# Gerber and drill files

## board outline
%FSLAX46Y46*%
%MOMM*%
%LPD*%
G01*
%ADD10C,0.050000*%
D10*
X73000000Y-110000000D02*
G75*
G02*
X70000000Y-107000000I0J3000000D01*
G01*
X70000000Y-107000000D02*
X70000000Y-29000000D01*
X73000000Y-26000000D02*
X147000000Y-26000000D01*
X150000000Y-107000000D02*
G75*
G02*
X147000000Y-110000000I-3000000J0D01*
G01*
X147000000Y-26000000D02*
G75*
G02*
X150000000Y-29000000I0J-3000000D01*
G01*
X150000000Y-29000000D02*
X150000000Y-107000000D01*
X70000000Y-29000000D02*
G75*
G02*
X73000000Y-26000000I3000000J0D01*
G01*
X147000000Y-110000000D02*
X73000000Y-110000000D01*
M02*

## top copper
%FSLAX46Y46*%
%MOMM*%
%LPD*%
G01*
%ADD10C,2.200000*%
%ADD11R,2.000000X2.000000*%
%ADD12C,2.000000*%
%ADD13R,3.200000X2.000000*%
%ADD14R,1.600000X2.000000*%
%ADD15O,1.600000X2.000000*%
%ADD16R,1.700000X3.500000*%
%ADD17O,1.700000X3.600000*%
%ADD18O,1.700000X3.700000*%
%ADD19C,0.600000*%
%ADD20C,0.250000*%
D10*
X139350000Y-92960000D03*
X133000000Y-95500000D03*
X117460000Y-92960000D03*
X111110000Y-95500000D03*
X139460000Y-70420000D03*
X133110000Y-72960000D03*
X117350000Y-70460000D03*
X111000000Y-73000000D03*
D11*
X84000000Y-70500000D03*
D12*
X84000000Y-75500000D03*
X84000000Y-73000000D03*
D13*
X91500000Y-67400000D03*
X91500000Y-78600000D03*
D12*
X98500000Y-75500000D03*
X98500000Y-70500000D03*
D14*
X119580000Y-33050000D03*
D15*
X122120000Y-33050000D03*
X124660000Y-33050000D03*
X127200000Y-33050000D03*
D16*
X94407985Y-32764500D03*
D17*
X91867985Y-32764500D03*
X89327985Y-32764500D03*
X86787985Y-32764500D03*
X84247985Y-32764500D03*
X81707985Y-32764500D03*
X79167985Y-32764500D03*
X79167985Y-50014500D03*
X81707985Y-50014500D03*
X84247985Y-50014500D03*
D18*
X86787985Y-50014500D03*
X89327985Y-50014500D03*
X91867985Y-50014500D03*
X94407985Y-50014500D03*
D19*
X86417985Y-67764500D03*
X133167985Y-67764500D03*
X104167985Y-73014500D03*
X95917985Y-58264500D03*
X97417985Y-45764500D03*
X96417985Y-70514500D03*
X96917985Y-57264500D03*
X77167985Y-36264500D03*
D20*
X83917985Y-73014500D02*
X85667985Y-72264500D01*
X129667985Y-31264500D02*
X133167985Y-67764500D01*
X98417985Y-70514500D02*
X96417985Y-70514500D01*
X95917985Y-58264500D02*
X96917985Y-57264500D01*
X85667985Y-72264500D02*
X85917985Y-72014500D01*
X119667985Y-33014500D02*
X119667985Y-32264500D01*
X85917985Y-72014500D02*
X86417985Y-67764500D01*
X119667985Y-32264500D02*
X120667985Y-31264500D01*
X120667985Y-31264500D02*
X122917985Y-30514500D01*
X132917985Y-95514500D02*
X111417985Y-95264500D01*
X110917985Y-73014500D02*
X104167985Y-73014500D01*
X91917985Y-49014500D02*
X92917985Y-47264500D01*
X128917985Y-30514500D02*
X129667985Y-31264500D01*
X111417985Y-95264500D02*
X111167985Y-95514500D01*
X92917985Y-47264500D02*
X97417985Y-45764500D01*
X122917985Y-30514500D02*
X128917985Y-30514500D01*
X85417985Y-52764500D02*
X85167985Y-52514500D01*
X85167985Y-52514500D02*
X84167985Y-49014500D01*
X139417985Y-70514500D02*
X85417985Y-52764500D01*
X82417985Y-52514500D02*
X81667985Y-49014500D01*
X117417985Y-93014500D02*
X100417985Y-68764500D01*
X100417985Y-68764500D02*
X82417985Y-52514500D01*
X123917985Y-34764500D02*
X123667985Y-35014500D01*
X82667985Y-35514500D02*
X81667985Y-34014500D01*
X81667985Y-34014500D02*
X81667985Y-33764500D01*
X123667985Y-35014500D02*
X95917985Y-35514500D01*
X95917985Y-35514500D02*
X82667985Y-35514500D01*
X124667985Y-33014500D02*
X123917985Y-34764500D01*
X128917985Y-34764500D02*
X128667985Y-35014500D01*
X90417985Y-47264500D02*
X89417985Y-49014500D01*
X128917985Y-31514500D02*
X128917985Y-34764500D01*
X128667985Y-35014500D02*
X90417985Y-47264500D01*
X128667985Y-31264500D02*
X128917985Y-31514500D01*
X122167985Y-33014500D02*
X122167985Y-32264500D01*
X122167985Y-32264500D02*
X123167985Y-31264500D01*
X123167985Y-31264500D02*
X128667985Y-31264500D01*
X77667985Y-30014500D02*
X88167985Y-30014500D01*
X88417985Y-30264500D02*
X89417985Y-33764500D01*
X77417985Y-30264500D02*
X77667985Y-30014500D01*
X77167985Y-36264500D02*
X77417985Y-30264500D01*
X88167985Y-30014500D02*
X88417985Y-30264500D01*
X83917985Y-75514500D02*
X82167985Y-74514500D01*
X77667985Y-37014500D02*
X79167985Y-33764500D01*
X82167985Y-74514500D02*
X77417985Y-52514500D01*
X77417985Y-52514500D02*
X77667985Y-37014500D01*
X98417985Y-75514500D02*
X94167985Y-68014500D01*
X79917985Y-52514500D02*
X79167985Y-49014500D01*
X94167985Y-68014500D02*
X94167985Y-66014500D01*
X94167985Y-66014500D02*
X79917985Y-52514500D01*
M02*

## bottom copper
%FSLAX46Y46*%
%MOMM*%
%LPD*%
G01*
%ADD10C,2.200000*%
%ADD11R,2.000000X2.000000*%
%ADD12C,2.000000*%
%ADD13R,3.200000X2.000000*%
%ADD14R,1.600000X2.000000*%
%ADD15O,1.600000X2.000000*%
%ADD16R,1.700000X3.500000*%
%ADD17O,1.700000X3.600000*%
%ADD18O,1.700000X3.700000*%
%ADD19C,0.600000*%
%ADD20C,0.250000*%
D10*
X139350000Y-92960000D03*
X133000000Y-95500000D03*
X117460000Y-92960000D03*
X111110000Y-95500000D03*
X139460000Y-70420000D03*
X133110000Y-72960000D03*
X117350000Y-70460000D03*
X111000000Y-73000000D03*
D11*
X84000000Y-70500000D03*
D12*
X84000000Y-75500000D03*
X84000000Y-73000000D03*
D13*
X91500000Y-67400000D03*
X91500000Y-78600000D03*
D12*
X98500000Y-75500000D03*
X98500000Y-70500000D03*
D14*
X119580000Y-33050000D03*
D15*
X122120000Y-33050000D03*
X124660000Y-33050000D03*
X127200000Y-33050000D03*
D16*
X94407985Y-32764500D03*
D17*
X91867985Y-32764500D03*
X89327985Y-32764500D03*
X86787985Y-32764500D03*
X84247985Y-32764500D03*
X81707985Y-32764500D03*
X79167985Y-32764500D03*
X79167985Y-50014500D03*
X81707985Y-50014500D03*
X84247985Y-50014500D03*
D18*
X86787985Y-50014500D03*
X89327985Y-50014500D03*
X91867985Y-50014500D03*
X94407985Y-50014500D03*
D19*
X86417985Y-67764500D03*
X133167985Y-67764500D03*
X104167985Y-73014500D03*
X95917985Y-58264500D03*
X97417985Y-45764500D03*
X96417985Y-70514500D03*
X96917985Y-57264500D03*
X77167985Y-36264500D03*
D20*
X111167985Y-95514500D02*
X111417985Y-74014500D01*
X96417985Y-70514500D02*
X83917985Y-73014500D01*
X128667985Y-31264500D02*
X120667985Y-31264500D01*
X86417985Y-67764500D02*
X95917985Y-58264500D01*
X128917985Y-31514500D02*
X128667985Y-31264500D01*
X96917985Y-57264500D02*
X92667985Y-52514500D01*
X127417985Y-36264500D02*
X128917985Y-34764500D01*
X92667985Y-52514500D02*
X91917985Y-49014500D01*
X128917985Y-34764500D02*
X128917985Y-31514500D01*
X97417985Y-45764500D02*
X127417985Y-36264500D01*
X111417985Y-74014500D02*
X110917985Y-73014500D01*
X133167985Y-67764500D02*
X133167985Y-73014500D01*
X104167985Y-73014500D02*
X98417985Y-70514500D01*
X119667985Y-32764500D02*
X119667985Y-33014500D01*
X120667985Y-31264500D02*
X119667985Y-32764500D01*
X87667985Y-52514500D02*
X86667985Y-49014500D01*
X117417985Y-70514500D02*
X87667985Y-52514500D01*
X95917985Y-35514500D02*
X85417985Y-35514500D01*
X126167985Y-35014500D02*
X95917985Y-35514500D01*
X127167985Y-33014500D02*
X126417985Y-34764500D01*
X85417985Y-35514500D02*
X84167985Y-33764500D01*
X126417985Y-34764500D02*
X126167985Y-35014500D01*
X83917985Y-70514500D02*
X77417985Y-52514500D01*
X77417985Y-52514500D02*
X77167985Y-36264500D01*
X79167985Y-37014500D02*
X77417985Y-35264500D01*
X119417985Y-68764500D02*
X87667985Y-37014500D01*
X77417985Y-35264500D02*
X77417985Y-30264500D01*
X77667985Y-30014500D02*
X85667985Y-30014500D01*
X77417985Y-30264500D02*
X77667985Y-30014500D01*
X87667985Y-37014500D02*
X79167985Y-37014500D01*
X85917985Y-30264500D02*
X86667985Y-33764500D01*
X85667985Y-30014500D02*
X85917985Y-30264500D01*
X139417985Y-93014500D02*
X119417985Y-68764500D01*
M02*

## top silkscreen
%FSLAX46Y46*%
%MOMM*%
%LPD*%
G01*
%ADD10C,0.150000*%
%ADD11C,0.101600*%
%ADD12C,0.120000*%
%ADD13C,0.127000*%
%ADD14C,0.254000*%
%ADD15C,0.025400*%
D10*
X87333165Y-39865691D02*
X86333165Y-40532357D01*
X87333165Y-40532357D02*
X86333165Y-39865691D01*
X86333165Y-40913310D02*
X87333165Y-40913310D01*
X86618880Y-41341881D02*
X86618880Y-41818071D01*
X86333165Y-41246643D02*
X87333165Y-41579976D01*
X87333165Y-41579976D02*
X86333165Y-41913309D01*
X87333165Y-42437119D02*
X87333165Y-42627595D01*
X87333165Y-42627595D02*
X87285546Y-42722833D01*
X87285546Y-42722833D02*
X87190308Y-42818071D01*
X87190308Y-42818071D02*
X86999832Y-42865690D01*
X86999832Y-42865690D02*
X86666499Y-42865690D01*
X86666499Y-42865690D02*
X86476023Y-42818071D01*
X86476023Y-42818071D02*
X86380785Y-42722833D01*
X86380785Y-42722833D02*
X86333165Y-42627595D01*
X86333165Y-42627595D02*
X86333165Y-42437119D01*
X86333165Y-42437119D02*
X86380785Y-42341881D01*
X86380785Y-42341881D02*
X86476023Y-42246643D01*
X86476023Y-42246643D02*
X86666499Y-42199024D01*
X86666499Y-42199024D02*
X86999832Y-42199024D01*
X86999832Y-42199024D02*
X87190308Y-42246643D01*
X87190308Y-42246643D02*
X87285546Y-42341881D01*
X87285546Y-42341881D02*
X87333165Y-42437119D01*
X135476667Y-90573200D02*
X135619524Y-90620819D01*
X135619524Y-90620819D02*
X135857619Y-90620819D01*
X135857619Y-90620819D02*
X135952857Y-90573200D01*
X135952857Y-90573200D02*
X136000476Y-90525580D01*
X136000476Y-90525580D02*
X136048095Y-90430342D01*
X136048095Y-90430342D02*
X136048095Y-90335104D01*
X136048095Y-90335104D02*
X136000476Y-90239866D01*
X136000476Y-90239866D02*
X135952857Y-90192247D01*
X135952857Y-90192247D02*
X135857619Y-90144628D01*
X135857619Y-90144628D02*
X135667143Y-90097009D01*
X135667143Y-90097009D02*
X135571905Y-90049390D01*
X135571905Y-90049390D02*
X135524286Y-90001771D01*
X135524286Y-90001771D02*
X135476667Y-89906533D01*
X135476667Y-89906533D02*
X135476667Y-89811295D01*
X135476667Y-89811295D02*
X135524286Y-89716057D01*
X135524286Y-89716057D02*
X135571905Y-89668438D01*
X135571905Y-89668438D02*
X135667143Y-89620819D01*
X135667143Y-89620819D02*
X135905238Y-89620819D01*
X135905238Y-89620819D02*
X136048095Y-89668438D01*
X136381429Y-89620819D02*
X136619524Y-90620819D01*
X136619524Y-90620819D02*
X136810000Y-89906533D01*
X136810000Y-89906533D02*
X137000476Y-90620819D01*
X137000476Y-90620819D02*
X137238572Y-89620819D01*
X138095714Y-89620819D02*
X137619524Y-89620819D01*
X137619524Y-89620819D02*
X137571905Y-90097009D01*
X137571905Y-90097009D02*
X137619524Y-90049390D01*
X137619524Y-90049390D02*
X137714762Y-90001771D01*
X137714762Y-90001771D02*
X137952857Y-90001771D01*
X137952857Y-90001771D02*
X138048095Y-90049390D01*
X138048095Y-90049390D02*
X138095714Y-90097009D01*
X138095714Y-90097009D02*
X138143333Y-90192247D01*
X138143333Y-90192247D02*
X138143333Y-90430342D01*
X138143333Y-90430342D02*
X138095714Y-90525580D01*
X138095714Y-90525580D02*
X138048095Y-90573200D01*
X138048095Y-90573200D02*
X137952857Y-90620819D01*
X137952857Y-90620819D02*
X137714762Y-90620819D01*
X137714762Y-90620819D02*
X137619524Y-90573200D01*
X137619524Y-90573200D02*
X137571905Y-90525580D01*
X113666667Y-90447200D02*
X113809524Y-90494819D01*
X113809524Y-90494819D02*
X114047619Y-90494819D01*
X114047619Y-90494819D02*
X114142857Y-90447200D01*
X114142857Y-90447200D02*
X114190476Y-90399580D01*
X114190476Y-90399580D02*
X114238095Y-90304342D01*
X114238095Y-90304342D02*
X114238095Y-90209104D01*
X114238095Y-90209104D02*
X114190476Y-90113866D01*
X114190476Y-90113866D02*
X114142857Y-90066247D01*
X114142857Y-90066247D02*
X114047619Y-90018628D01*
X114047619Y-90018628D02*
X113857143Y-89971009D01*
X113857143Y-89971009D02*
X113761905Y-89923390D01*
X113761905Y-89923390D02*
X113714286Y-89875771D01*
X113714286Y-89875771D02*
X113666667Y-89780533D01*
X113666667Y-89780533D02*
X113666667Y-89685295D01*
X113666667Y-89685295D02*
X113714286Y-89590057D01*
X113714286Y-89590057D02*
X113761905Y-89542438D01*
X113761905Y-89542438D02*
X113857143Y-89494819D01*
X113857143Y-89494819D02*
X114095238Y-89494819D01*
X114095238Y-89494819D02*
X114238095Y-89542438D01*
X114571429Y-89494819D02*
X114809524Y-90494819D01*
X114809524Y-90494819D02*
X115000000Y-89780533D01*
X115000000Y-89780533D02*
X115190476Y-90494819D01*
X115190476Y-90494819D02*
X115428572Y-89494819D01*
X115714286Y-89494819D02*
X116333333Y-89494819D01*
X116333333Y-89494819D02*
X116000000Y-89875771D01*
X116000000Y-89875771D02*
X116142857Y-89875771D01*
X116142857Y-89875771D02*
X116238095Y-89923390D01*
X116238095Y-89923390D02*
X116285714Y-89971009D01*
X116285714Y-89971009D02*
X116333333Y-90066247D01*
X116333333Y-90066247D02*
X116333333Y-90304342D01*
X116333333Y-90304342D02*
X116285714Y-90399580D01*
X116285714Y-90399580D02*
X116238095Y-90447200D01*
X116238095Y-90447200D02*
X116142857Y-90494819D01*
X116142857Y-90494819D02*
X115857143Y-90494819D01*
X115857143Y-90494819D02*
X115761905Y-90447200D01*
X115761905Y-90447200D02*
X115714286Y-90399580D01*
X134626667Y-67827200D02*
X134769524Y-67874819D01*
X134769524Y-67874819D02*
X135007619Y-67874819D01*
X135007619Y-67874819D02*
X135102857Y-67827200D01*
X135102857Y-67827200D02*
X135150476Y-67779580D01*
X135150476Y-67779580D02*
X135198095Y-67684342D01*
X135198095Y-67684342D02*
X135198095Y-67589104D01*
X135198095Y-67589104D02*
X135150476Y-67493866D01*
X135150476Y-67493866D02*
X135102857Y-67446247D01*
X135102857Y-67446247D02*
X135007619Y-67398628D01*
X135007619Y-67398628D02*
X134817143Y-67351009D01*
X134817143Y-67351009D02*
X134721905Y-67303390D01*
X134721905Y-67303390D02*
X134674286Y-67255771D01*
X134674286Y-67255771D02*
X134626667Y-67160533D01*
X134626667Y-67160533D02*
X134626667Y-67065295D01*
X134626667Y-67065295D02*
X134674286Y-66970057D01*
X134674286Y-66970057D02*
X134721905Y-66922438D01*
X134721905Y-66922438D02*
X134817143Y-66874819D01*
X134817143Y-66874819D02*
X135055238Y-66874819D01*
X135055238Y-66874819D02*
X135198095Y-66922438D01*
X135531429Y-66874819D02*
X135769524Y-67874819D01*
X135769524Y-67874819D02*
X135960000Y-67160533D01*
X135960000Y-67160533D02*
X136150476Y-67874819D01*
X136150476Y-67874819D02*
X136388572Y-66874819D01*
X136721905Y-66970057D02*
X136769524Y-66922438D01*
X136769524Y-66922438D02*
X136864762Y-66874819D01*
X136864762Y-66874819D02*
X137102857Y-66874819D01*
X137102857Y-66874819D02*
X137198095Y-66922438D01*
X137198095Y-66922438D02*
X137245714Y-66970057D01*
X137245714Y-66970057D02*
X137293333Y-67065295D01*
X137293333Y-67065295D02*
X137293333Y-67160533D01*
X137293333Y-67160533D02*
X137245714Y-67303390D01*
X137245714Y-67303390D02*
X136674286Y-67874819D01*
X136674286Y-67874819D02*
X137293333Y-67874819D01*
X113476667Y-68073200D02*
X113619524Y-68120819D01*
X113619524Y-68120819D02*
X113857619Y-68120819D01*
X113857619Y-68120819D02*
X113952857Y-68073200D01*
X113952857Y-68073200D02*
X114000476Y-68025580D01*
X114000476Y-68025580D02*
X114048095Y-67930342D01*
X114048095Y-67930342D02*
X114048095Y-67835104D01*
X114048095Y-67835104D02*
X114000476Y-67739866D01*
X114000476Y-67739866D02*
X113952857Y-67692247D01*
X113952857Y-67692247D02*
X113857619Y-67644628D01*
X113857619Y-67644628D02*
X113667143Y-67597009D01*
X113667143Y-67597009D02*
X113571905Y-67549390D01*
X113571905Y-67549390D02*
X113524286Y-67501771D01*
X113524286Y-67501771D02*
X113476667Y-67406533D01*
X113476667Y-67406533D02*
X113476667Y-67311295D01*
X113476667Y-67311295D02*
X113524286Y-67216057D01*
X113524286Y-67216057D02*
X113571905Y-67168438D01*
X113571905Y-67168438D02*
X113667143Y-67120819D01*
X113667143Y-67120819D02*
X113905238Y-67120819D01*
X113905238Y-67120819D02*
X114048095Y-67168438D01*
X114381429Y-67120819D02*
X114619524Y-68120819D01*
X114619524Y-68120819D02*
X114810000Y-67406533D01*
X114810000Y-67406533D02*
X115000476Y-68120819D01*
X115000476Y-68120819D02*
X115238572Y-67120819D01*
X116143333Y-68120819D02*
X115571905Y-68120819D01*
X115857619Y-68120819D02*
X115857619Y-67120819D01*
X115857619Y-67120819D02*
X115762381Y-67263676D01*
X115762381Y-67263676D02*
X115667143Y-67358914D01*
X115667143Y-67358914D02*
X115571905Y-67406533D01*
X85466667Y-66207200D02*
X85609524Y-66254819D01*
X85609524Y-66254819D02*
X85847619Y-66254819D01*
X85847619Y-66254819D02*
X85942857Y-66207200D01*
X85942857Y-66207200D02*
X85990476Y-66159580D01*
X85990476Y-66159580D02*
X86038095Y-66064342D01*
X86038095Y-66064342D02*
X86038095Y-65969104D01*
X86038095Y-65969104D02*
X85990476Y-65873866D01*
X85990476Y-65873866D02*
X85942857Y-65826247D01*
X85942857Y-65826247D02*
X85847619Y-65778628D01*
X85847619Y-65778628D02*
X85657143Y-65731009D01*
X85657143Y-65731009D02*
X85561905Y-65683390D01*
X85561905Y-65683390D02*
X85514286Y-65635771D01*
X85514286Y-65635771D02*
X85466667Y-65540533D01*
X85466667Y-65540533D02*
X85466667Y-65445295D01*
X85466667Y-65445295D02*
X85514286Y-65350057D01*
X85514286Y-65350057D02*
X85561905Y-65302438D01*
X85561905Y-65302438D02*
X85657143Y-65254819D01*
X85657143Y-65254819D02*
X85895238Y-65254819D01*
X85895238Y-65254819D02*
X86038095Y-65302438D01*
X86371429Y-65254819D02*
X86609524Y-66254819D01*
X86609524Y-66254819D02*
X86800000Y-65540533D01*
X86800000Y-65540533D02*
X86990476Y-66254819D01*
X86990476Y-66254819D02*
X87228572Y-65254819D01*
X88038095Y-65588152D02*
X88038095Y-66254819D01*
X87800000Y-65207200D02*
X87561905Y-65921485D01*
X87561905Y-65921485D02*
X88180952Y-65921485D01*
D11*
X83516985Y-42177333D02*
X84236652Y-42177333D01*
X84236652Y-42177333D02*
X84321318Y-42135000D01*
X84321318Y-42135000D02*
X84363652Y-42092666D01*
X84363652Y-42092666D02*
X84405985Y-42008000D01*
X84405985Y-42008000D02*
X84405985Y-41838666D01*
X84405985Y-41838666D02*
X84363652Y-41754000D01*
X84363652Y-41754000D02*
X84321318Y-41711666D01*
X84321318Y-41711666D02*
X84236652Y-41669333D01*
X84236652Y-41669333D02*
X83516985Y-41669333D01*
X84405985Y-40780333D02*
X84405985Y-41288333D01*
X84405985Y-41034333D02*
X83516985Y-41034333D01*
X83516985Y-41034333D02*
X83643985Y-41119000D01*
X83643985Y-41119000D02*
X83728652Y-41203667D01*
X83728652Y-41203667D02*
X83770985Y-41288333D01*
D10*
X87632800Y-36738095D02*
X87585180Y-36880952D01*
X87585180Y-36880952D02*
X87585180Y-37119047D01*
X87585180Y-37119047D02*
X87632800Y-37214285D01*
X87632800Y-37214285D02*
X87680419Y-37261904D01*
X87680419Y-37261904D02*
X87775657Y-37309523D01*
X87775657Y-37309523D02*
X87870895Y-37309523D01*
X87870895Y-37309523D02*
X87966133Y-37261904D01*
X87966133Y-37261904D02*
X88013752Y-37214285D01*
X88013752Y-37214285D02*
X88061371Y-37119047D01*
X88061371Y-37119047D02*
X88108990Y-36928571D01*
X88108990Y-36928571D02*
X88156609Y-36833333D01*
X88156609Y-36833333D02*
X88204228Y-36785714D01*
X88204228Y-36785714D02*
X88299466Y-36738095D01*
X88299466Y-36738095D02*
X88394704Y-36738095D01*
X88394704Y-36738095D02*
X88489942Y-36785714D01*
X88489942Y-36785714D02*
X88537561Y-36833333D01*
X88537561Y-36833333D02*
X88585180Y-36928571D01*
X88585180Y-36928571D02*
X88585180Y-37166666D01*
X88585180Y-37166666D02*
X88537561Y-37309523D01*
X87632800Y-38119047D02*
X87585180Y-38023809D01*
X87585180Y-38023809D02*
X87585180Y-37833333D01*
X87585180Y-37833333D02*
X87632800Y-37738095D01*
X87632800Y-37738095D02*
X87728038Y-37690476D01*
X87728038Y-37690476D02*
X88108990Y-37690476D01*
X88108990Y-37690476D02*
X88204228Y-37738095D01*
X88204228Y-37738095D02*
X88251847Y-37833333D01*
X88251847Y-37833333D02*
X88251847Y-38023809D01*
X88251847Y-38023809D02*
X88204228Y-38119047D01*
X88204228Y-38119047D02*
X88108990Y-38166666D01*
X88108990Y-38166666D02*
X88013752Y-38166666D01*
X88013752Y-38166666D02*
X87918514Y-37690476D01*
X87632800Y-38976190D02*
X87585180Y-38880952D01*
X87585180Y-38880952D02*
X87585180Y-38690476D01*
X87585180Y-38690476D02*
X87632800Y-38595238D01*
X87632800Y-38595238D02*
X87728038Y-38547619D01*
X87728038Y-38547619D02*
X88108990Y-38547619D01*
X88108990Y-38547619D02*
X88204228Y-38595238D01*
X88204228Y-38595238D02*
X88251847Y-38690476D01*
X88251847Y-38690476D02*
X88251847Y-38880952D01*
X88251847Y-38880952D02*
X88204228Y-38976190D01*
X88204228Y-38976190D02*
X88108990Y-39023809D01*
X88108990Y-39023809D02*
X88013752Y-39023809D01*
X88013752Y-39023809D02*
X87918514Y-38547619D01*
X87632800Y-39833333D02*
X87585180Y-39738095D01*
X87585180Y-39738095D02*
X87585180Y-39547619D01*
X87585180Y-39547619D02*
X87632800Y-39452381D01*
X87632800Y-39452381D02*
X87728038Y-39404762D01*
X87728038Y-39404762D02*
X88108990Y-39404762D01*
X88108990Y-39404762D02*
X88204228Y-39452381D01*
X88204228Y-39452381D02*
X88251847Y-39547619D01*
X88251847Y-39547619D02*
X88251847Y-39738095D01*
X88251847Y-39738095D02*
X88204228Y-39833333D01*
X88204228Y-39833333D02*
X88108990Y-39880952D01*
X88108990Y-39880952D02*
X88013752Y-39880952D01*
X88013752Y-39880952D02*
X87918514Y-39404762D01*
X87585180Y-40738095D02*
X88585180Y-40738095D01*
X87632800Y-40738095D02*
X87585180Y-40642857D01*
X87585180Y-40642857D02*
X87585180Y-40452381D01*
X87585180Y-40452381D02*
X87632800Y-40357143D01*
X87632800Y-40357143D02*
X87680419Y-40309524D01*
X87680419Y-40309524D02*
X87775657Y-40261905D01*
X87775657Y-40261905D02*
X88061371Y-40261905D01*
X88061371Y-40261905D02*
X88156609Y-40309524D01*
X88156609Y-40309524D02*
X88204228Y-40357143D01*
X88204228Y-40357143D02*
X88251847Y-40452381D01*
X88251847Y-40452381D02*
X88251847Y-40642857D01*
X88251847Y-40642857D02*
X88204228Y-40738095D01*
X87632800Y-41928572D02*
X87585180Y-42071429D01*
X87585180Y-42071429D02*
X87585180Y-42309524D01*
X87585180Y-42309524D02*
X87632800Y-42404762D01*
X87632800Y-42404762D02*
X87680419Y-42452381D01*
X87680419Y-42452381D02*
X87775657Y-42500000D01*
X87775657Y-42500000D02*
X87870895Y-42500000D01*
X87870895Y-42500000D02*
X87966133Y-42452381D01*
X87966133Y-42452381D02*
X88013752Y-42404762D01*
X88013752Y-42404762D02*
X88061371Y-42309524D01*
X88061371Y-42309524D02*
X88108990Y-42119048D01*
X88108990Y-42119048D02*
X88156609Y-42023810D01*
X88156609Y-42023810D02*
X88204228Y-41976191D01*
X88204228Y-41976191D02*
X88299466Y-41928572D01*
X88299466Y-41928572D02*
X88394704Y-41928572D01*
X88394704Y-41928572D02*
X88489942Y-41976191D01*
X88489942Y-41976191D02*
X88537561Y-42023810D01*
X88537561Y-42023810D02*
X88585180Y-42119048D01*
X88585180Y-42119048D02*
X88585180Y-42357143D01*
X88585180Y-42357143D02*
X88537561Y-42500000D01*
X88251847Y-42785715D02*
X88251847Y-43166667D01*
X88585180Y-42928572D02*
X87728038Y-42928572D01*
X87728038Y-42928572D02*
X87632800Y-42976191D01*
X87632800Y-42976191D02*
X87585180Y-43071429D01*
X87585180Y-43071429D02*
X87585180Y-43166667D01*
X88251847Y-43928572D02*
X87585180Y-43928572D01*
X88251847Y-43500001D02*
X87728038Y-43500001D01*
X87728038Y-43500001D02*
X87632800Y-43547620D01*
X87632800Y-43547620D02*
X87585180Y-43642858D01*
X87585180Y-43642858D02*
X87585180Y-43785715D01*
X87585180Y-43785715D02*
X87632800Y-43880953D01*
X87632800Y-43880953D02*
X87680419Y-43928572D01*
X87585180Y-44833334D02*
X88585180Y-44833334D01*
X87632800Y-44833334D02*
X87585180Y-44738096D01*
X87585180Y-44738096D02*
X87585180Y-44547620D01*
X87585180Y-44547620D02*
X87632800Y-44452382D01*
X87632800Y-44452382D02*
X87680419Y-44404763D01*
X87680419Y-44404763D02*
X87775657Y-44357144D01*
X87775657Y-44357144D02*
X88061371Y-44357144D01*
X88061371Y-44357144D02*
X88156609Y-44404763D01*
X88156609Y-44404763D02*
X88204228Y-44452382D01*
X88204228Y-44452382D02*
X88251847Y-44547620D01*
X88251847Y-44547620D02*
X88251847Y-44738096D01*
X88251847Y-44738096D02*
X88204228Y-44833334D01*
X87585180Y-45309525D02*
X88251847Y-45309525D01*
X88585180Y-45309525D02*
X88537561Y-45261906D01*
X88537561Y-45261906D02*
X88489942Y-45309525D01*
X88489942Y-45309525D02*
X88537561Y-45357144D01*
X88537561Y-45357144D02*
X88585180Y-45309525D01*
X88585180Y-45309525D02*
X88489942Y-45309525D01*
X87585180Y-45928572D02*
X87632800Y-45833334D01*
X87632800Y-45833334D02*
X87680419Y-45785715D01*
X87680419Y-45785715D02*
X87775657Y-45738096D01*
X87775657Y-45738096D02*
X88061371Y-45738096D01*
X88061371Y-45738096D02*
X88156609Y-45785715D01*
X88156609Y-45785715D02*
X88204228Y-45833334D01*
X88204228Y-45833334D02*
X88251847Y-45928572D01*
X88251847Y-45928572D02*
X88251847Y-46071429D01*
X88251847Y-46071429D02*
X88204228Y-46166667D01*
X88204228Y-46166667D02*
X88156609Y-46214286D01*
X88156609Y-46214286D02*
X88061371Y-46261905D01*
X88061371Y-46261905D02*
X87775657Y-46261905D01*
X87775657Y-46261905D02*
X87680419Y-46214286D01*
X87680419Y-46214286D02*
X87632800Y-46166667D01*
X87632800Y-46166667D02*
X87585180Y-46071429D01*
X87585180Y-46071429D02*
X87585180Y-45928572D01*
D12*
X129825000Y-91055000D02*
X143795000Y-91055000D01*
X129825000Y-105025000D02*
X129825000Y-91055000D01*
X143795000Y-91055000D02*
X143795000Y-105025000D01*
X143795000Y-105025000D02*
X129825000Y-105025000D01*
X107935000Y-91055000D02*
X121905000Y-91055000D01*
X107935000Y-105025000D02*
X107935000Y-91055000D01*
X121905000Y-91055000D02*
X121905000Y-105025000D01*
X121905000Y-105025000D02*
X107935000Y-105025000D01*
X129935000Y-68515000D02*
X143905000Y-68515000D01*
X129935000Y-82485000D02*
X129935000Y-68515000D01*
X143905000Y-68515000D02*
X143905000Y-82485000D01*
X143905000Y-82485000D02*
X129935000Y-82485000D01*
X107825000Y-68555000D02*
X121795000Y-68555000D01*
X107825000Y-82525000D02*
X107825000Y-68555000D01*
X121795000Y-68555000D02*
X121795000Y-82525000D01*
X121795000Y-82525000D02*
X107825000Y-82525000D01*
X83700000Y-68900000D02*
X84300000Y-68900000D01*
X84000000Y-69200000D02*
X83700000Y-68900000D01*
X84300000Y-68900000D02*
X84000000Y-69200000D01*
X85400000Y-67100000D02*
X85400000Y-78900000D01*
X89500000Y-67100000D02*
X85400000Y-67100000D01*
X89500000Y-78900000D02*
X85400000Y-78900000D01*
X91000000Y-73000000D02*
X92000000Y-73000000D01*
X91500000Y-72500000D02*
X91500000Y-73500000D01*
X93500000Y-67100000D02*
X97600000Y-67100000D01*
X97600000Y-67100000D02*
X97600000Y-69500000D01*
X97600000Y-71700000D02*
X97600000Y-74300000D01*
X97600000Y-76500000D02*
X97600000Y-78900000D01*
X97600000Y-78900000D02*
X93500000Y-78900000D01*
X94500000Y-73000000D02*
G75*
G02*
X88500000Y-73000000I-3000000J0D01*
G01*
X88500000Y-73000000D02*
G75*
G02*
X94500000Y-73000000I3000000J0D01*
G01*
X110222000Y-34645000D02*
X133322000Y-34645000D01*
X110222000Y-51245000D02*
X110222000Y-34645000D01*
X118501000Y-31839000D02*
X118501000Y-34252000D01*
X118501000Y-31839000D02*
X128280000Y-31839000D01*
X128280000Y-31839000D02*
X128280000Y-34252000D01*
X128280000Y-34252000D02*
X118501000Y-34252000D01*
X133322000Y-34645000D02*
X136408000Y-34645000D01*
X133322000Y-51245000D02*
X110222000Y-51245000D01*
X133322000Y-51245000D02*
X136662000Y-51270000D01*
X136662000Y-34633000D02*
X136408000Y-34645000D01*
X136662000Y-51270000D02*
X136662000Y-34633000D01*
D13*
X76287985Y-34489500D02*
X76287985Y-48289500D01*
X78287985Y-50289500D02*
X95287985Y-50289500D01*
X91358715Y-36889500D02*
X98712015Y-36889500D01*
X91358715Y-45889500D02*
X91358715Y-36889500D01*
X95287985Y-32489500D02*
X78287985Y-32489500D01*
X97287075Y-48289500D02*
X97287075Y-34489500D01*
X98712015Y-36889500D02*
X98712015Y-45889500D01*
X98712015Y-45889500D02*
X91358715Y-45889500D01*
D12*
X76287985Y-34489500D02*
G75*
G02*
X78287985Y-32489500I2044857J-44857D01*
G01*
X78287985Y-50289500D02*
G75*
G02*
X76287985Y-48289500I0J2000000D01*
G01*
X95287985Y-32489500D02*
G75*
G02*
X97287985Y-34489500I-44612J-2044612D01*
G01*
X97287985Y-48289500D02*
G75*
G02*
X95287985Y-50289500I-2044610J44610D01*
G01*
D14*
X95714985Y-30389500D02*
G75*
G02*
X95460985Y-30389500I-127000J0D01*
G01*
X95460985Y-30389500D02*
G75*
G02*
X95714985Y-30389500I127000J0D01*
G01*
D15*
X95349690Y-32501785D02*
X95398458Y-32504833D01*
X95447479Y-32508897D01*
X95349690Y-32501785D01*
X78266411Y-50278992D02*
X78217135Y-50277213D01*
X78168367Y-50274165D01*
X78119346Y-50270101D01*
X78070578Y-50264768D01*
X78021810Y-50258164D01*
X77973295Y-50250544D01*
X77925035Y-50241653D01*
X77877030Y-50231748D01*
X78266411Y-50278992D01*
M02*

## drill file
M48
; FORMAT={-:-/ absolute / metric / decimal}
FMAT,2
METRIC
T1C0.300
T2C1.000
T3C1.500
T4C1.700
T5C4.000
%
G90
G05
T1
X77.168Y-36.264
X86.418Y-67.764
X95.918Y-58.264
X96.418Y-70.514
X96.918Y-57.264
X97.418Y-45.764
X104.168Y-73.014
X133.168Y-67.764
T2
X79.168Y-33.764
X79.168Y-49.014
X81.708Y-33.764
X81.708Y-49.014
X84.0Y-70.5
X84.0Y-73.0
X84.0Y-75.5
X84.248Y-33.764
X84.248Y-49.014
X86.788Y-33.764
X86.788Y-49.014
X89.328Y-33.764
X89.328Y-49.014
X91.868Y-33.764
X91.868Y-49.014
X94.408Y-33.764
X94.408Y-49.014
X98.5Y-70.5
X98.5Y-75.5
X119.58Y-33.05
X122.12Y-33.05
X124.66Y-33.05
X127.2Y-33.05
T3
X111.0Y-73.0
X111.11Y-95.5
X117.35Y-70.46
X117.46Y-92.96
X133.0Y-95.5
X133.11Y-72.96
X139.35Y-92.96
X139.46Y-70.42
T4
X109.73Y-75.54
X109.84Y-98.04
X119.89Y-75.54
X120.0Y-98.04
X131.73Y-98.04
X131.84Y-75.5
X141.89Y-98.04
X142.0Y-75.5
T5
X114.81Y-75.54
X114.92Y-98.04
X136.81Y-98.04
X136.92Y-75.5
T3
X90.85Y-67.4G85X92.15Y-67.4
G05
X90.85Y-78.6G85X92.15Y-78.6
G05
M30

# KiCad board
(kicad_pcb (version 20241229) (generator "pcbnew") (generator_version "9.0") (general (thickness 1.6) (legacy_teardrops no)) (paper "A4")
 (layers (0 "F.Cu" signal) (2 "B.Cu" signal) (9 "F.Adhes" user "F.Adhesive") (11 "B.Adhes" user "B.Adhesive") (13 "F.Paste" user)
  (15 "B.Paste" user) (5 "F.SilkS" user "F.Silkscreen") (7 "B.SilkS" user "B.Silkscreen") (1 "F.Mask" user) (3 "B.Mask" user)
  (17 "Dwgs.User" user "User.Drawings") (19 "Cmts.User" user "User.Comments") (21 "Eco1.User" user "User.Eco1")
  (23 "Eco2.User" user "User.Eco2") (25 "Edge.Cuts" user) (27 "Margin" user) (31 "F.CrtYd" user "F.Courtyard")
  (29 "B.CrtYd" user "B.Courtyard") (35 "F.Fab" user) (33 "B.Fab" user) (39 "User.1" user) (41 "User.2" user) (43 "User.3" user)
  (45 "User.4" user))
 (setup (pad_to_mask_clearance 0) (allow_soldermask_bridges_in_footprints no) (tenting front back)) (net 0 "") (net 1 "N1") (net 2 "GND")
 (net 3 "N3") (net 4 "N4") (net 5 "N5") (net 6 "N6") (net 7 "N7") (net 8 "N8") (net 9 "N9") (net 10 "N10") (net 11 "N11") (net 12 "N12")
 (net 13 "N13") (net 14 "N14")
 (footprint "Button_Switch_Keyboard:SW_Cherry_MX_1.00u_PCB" (layer "F.Cu") (at 139.35 92.96)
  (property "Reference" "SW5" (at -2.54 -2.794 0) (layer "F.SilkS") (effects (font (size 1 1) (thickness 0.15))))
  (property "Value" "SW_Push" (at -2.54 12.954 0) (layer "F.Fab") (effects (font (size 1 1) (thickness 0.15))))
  (fp_line (start -9.525 -1.905) (end 4.445 -1.905) (stroke (width 0.12) (type solid)) (layer "F.SilkS"))
  (fp_line (start -9.525 12.065) (end -9.525 -1.905) (stroke (width 0.12) (type solid)) (layer "F.SilkS"))
  (fp_line (start 4.445 -1.905) (end 4.445 12.065) (stroke (width 0.12) (type solid)) (layer "F.SilkS"))
  (fp_line (start 4.445 12.065) (end -9.525 12.065) (stroke (width 0.12) (type solid)) (layer "F.SilkS"))
  (pad "" np_thru_hole circle (at -7.62 5.08) (size 1.7 1.7) (drill 1.7) (layers "*.Cu" "*.Mask"))
  (pad "" np_thru_hole circle (at -2.54 5.08) (size 4 4) (drill 4) (layers "*.Cu" "*.Mask"))
  (pad "" np_thru_hole circle (at 2.54 5.08) (size 1.7 1.7) (drill 1.7) (layers "*.Cu" "*.Mask"))
  (pad "1" thru_hole circle (at 0 0) (size 2.2 2.2) (drill 1.5) (layers "*.Cu" "*.Mask") (remove_unused_layers no) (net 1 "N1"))
  (pad "2" thru_hole circle (at -6.35 2.54) (size 2.2 2.2) (drill 1.5) (layers "*.Cu" "*.Mask") (remove_unused_layers no) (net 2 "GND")))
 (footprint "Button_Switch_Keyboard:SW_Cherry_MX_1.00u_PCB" (layer "F.Cu") (at 117.46 92.96)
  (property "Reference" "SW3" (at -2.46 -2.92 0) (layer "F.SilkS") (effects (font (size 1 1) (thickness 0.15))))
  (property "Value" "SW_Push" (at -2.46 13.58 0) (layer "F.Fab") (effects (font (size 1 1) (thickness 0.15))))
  (fp_line (start -9.525 -1.905) (end 4.445 -1.905) (stroke (width 0.12) (type solid)) (layer "F.SilkS"))
  (fp_line (start -9.525 12.065) (end -9.525 -1.905) (stroke (width 0.12) (type solid)) (layer "F.SilkS"))
  (fp_line (start 4.445 -1.905) (end 4.445 12.065) (stroke (width 0.12) (type solid)) (layer "F.SilkS"))
  (fp_line (start 4.445 12.065) (end -9.525 12.065) (stroke (width 0.12) (type solid)) (layer "F.SilkS"))
  (pad "" np_thru_hole circle (at -7.62 5.08) (size 1.7 1.7) (drill 1.7) (layers "*.Cu" "*.Mask"))
  (pad "" np_thru_hole circle (at -2.54 5.08) (size 4 4) (drill 4) (layers "*.Cu" "*.Mask"))
  (pad "" np_thru_hole circle (at 2.54 5.08) (size 1.7 1.7) (drill 1.7) (layers "*.Cu" "*.Mask"))
  (pad "1" thru_hole circle (at 0 0) (size 2.2 2.2) (drill 1.5) (layers "*.Cu" "*.Mask") (remove_unused_layers no) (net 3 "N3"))
  (pad "2" thru_hole circle (at -6.35 2.54) (size 2.2 2.2) (drill 1.5) (layers "*.Cu" "*.Mask") (remove_unused_layers no) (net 2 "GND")))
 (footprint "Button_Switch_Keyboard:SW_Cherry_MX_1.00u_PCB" (layer "F.Cu") (at 139.46 70.42)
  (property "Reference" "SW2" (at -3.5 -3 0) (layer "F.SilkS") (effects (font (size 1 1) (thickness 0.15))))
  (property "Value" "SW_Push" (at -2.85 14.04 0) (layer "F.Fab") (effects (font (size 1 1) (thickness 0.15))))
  (fp_line (start -9.525 -1.905) (end 4.445 -1.905) (stroke (width 0.12) (type solid)) (layer "F.SilkS"))
  (fp_line (start -9.525 12.065) (end -9.525 -1.905) (stroke (width 0.12) (type solid)) (layer "F.SilkS"))
  (fp_line (start 4.445 -1.905) (end 4.445 12.065) (stroke (width 0.12) (type solid)) (layer "F.SilkS"))
  (fp_line (start 4.445 12.065) (end -9.525 12.065) (stroke (width 0.12) (type solid)) (layer "F.SilkS"))
  (pad "" np_thru_hole circle (at -7.62 5.08) (size 1.7 1.7) (drill 1.7) (layers "*.Cu" "*.Mask"))
  (pad "" np_thru_hole circle (at -2.54 5.08) (size 4 4) (drill 4) (layers "*.Cu" "*.Mask"))
  (pad "" np_thru_hole circle (at 2.54 5.08) (size 1.7 1.7) (drill 1.7) (layers "*.Cu" "*.Mask"))
  (pad "1" thru_hole circle (at 0 0) (size 2.2 2.2) (drill 1.5) (layers "*.Cu" "*.Mask") (remove_unused_layers no) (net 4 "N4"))
  (pad "2" thru_hole circle (at -6.35 2.54) (size 2.2 2.2) (drill 1.5) (layers "*.Cu" "*.Mask") (remove_unused_layers no) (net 2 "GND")))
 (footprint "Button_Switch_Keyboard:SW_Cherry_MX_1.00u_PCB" (layer "F.Cu") (at 117.35 70.46)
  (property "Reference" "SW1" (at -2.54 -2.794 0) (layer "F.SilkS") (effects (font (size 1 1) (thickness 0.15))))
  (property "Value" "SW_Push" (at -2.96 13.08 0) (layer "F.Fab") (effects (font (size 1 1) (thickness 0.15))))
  (fp_line (start -9.525 -1.905) (end 4.445 -1.905) (stroke (width 0.12) (type solid)) (layer "F.SilkS"))
  (fp_line (start -9.525 12.065) (end -9.525 -1.905) (stroke (width 0.12) (type solid)) (layer "F.SilkS"))
  (fp_line (start 4.445 -1.905) (end 4.445 12.065) (stroke (width 0.12) (type solid)) (layer "F.SilkS"))
  (fp_line (start 4.445 12.065) (end -9.525 12.065) (stroke (width 0.12) (type solid)) (layer "F.SilkS"))
  (pad "" np_thru_hole circle (at -7.62 5.08) (size 1.7 1.7) (drill 1.7) (layers "*.Cu" "*.Mask"))
  (pad "" np_thru_hole circle (at -2.54 5.08) (size 4 4) (drill 4) (layers "*.Cu" "*.Mask"))
  (pad "" np_thru_hole circle (at 2.54 5.08) (size 1.7 1.7) (drill 1.7) (layers "*.Cu" "*.Mask"))
  (pad "1" thru_hole circle (at 0 0) (size 2.2 2.2) (drill 1.5) (layers "*.Cu" "*.Mask") (remove_unused_layers no) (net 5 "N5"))
  (pad "2" thru_hole circle (at -6.35 2.54) (size 2.2 2.2) (drill 1.5) (layers "*.Cu" "*.Mask") (remove_unused_layers no) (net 2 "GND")))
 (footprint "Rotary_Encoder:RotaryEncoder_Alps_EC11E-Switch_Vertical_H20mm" (layer "F.Cu") (at 84 70.5)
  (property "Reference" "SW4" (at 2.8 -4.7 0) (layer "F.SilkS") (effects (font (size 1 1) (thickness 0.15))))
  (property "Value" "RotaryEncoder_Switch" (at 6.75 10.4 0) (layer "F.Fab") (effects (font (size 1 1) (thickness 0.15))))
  (fp_line (start -0.3 -1.6) (end 0.3 -1.6) (stroke (width 0.12) (type solid)) (layer "F.SilkS"))
  (fp_line (start 0 -1.3) (end -0.3 -1.6) (stroke (width 0.12) (type solid)) (layer "F.SilkS"))
  (fp_line (start 0.3 -1.6) (end 0 -1.3) (stroke (width 0.12) (type solid)) (layer "F.SilkS"))
  (fp_line (start 1.4 -3.4) (end 1.4 8.4) (stroke (width 0.12) (type solid)) (layer "F.SilkS"))
  (fp_line (start 5.5 -3.4) (end 1.4 -3.4) (stroke (width 0.12) (type solid)) (layer "F.SilkS"))
  (fp_line (start 5.5 8.4) (end 1.4 8.4) (stroke (width 0.12) (type solid)) (layer "F.SilkS"))
  (fp_line (start 7 2.5) (end 8 2.5) (stroke (width 0.12) (type solid)) (layer "F.SilkS"))
  (fp_line (start 7.5 2) (end 7.5 3) (stroke (width 0.12) (type solid)) (layer "F.SilkS"))
  (fp_line (start 9.5 -3.4) (end 13.6 -3.4) (stroke (width 0.12) (type solid)) (layer "F.SilkS"))
  (fp_line (start 13.6 -3.4) (end 13.6 -1) (stroke (width 0.12) (type solid)) (layer "F.SilkS"))
  (fp_line (start 13.6 1.2) (end 13.6 3.8) (stroke (width 0.12) (type solid)) (layer "F.SilkS"))
  (fp_line (start 13.6 6) (end 13.6 8.4) (stroke (width 0.12) (type solid)) (layer "F.SilkS"))
  (fp_line (start 13.6 8.4) (end 9.5 8.4) (stroke (width 0.12) (type solid)) (layer "F.SilkS"))
  (fp_circle (center 7.5 2.5) (end 10.5 2.5) (stroke (width 0.12) (type solid)) (fill no) (layer "F.SilkS"))
  (pad "A" thru_hole rect (at 0 0) (size 2 2) (drill 1) (layers "*.Cu" "*.Mask") (remove_unused_layers no) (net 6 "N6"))
  (pad "B" thru_hole circle (at 0 5) (size 2 2) (drill 1) (layers "*.Cu" "*.Mask") (remove_unused_layers no) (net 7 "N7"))
  (pad "C" thru_hole circle (at 0 2.5) (size 2 2) (drill 1) (layers "*.Cu" "*.Mask") (remove_unused_layers no) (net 2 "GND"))
  (pad "MP" thru_hole rect (at 7.5 -3.1) (size 3.2 2) (drill oval 2.8 1.5) (layers "*.Cu" "*.Mask") (remove_unused_layers no))
  (pad "MP" thru_hole rect (at 7.5 8.1) (size 3.2 2) (drill oval 2.8 1.5) (layers "*.Cu" "*.Mask") (remove_unused_layers no))
  (pad "S1" thru_hole circle (at 14.5 5) (size 2 2) (drill 1) (layers "*.Cu" "*.Mask") (remove_unused_layers no) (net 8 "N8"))
  (pad "S2" thru_hole circle (at 14.5 0) (size 2 2) (drill 1) (layers "*.Cu" "*.Mask") (remove_unused_layers no) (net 2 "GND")))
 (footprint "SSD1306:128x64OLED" (layer "F.Cu") (at 123.2 43.65)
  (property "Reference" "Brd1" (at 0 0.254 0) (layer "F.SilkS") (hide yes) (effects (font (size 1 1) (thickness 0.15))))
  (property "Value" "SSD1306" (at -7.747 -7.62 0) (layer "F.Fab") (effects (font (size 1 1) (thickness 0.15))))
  (fp_line (start -12.978 -9.005) (end 10.122 -9.005) (stroke (width 0.12) (type solid)) (layer "F.SilkS"))
  (fp_line (start -12.978 7.595) (end -12.978 -9.005) (stroke (width 0.12) (type solid)) (layer "F.SilkS"))
  (fp_line (start -4.699 -11.811) (end -4.699 -9.398) (stroke (width 0.12) (type solid)) (layer "F.SilkS"))
  (fp_line (start -4.699 -11.811) (end 5.08 -11.811) (stroke (width 0.12) (type solid)) (layer "F.SilkS"))
  (fp_line (start 5.08 -11.811) (end 5.08 -9.398) (stroke (width 0.12) (type solid)) (layer "F.SilkS"))
  (fp_line (start 5.08 -9.398) (end -4.699 -9.398) (stroke (width 0.12) (type solid)) (layer "F.SilkS"))
  (fp_line (start 10.122 -9.005) (end 13.208 -9.005) (stroke (width 0.12) (type solid)) (layer "F.SilkS"))
  (fp_line (start 10.122 7.595) (end -12.978 7.595) (stroke (width 0.12) (type solid)) (layer "F.SilkS"))
  (fp_line (start 10.122 7.595) (end 13.462 7.62) (stroke (width 0.12) (type solid)) (layer "F.SilkS"))
  (fp_line (start 13.462 -9.017) (end 13.208 -9.005) (stroke (width 0.12) (type solid)) (layer "F.SilkS"))
  (fp_line (start 13.462 7.62) (end 13.462 -9.017) (stroke (width 0.12) (type solid)) (layer "F.SilkS"))
  (pad "1" thru_hole rect (at -3.62 -10.6 90) (size 2 1.6) (drill 1) (layers "*.Cu" "*.Mask") (remove_unused_layers no) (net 2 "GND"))
  (pad "2" thru_hole oval (at -1.08 -10.6 90) (size 2 1.6) (drill 1) (layers "*.Cu" "*.Mask") (remove_unused_layers no) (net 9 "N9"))
  (pad "3" thru_hole oval (at 1.46 -10.6 90) (size 2 1.6) (drill 1) (layers "*.Cu" "*.Mask") (remove_unused_layers no) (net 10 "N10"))
  (pad "4" thru_hole oval (at 4 -10.6 90) (size 2 1.6) (drill 1) (layers "*.Cu" "*.Mask") (remove_unused_layers no) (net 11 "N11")))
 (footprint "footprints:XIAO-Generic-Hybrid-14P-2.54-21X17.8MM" (layer "F.Cu") (at 86.787985 41.3895 -90)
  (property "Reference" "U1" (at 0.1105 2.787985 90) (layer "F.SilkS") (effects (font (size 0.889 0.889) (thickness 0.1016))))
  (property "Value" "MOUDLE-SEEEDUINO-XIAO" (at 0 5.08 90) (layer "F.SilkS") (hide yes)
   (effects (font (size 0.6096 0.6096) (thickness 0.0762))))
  (fp_line (start -6.9 10.5) (end 6.9 10.5) (stroke (width 0.127) (type solid)) (layer "F.SilkS"))
  (fp_line (start 8.9 8.5) (end 8.9 -8.5) (stroke (width 0.127) (type solid)) (layer "F.SilkS"))
  (fp_line (start -4.5 -4.57073) (end -4.5 -11.92403) (stroke (width 0.127) (type solid)) (layer "F.SilkS"))
  (fp_line (start 4.5 -4.57073) (end -4.5 -4.57073) (stroke (width 0.127) (type solid)) (layer "F.SilkS"))
  (fp_line (start -8.9 -8.5) (end -8.9 8.5) (stroke (width 0.127) (type solid)) (layer "F.SilkS"))
  (fp_line (start 6.9 -10.49909) (end -6.9 -10.49909) (stroke (width 0.127) (type solid)) (layer "F.SilkS"))
  (fp_line (start -4.5 -11.92403) (end 4.5 -11.92403) (stroke (width 0.127) (type solid)) (layer "F.SilkS"))
  (fp_line (start 4.5 -11.92403) (end 4.5 -4.57073) (stroke (width 0.127) (type solid)) (layer "F.SilkS"))
  (fp_arc (start -6.9 10.5) (mid -8.301423 9.901423) (end -8.9 8.5) (stroke (width 0.12) (type solid)) (layer "F.SilkS"))
  (fp_arc (start 8.9 8.5) (mid 8.314214 9.914214) (end 6.9 10.5) (stroke (width 0.12) (type solid)) (layer "F.SilkS"))
  (fp_arc (start -8.9 -8.5) (mid -8.301491 -9.901491) (end -6.9 -10.5) (stroke (width 0.12) (type solid)) (layer "F.SilkS"))
  (fp_arc (start 6.9 -10.5) (mid 8.301491 -9.901491) (end 8.9 -8.5) (stroke (width 0.12) (type solid)) (layer "F.SilkS"))
  (fp_circle (center -11 -8.8) (end -11 -9.054) (stroke (width 0) (type solid)) (fill yes) (layer "F.SilkS"))
  (fp_poly
   (pts (xy -8.887715 -8.561705) (xy -8.884667 -8.610473) (xy -8.880603 -8.659494)) (stroke (width 0.0254) (type solid)) (fill no)
   (layer "F.SilkS"))
  (fp_poly
   (pts (xy 8.889492 8.521574) (xy 8.887713 8.57085) (xy 8.884665 8.619618) (xy 8.880601 8.668639) (xy 8.875268 8.717407)
    (xy 8.868664 8.766175) (xy 8.861044 8.81469) (xy 8.852153 8.86295) (xy 8.842248 8.910955))
   (stroke (width 0.0254) (type solid)) (fill no) (layer "F.SilkS"))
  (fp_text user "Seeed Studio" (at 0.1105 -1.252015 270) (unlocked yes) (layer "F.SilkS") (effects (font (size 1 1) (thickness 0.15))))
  (pad "1" thru_hole rect (at -7.625 -7.62 270) (size 3.5 1.7) (drill 1 (offset -1 0)) (layers "*.Cu" "*.Mask") (remove_unused_layers no)
   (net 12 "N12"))
  (pad "2" thru_hole oval (at -7.625 -5.08 270) (size 3.6 1.7) (drill 1 (offset -1 0)) (layers "*.Cu" "*.Mask") (remove_unused_layers no)
   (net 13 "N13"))
  (pad "3" thru_hole oval (at -7.625 -2.54 270) (size 3.6 1.7) (drill 1 (offset -1 0)) (layers "*.Cu" "*.Mask") (remove_unused_layers no)
   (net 6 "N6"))
  (pad "4" thru_hole oval (at -7.625 0 270) (size 3.6 1.7) (drill 1 (offset -1 0)) (layers "*.Cu" "*.Mask") (remove_unused_layers no)
   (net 1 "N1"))
  (pad "5" thru_hole oval (at -7.625 2.54 270) (size 3.6 1.7) (drill 1 (offset -1 0)) (layers "*.Cu" "*.Mask") (remove_unused_layers no)
   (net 11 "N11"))
  (pad "6" thru_hole oval (at -7.625 5.08 90) (size 3.6 1.7) (drill 1 (offset 1 0)) (layers "*.Cu" "*.Mask") (remove_unused_layers no)
   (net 10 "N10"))
  (pad "7" thru_hole oval (at -7.625 7.62 270) (size 3.6 1.7) (drill 1 (offset -1 0)) (layers "*.Cu" "*.Mask") (remove_unused_layers no)
   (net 7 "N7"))
  (pad "8" thru_hole oval (at 7.625 7.62 270) (size 3.6 1.7) (drill 1 (offset 1 0)) (layers "*.Cu" "*.Mask") (remove_unused_layers no)
   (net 8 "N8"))
  (pad "9" thru_hole oval (at 7.625 5.08 270) (size 3.6 1.7) (drill 1 (offset 1 0)) (layers "*.Cu" "*.Mask") (remove_unused_layers no)
   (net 3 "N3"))
  (pad "10" thru_hole oval (at 7.625 2.54 270) (size 3.6 1.7) (drill 1 (offset 1 0)) (layers "*.Cu" "*.Mask") (remove_unused_layers no)
   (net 4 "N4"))
  (pad "11" thru_hole oval (at 7.625 0 270) (size 3.7 1.7) (drill 1 (offset 1 0)) (layers "*.Cu" "*.Mask") (remove_unused_layers no)
   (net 5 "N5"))
  (pad "12" thru_hole oval (at 7.625 -2.54 270) (size 3.7 1.7) (drill 1 (offset 1 0)) (layers "*.Cu" "*.Mask") (remove_unused_layers no)
   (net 9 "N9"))
  (pad "13" thru_hole oval (at 7.625 -5.08 270) (size 3.7 1.7) (drill 1 (offset 1 0)) (layers "*.Cu" "*.Mask") (remove_unused_layers no)
   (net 2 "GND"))
  (pad "14" thru_hole oval (at 7.625 -7.62 270) (size 3.7 1.7) (drill 1 (offset 1 0)) (layers "*.Cu" "*.Mask") (remove_unused_layers no)
   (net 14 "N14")))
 (gr_arc (start 73 110) (mid 70.87868 109.12132) (end 70 107) (stroke (width 0.05) (type default)) (layer "Edge.Cuts"))
 (gr_line (start 70 107) (end 70 29) (stroke (width 0.05) (type default)) (layer "Edge.Cuts"))
 (gr_line (start 73 26) (end 147 26) (stroke (width 0.05) (type default)) (layer "Edge.Cuts"))
 (gr_arc (start 150 107) (mid 149.12132 109.12132) (end 147 110) (stroke (width 0.05) (type default)) (layer "Edge.Cuts"))
 (gr_arc (start 147 26) (mid 149.12132 26.87868) (end 150 29) (stroke (width 0.05) (type default)) (layer "Edge.Cuts"))
 (gr_line (start 150 29) (end 150 107) (stroke (width 0.05) (type default)) (layer "Edge.Cuts"))
 (gr_arc (start 70 29) (mid 70.87868 26.87868) (end 73 26) (stroke (width 0.05) (type default)) (layer "Edge.Cuts"))
 (gr_line (start 147 110) (end 73 110) (stroke (width 0.05) (type default)) (layer "Edge.Cuts"))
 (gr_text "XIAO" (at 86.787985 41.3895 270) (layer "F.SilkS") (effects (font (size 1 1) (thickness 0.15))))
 (segment (start 83.917985 73.0145) (end 85.667985 72.2645) (width 0.25) (layer "F.Cu") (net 2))
 (segment (start 129.667985 31.2645) (end 133.167985 67.7645) (width 0.25) (layer "F.Cu") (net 2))
 (segment (start 98.417985 70.5145) (end 96.417985 70.5145) (width 0.25) (layer "F.Cu") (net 2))
 (segment (start 95.917985 58.2645) (end 96.917985 57.2645) (width 0.25) (layer "F.Cu") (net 2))
 (segment (start 85.667985 72.2645) (end 85.917985 72.0145) (width 0.25) (layer "F.Cu") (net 2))
 (segment (start 119.667985 33.0145) (end 119.667985 32.2645) (width 0.25) (layer "F.Cu") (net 2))
 (segment (start 85.917985 72.0145) (end 86.417985 67.7645) (width 0.25) (layer "F.Cu") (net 2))
 (segment (start 119.667985 32.2645) (end 120.667985 31.2645) (width 0.25) (layer "F.Cu") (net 2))
 (segment (start 120.667985 31.2645) (end 122.917985 30.5145) (width 0.25) (layer "F.Cu") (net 2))
 (segment (start 132.917985 95.5145) (end 111.417985 95.2645) (width 0.25) (layer "F.Cu") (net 2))
 (segment (start 110.917985 73.0145) (end 104.167985 73.0145) (width 0.25) (layer "F.Cu") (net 2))
 (segment (start 91.917985 49.0145) (end 92.917985 47.2645) (width 0.25) (layer "F.Cu") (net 2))
 (segment (start 128.917985 30.5145) (end 129.667985 31.2645) (width 0.25) (layer "F.Cu") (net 2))
 (segment (start 111.417985 95.2645) (end 111.167985 95.5145) (width 0.25) (layer "F.Cu") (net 2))
 (segment (start 92.917985 47.2645) (end 97.417985 45.7645) (width 0.25) (layer "F.Cu") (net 2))
 (segment (start 122.917985 30.5145) (end 128.917985 30.5145) (width 0.25) (layer "F.Cu") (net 2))
 (via (at 86.417985 67.7645) (size 0.6) (drill 0.3) (layers "F.Cu" "B.Cu") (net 2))
 (via (at 133.167985 67.7645) (size 0.6) (drill 0.3) (layers "F.Cu" "B.Cu") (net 2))
 (via (at 104.167985 73.0145) (size 0.6) (drill 0.3) (layers "F.Cu" "B.Cu") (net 2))
 (via (at 95.917985 58.2645) (size 0.6) (drill 0.3) (layers "F.Cu" "B.Cu") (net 2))
 (via (at 97.417985 45.7645) (size 0.6) (drill 0.3) (layers "F.Cu" "B.Cu") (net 2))
 (via (at 96.417985 70.5145) (size 0.6) (drill 0.3) (layers "F.Cu" "B.Cu") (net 2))
 (via (at 96.917985 57.2645) (size 0.6) (drill 0.3) (layers "F.Cu" "B.Cu") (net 2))
 (segment (start 111.167985 95.5145) (end 111.417985 74.0145) (width 0.25) (layer "B.Cu") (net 2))
 (segment (start 96.417985 70.5145) (end 83.917985 73.0145) (width 0.25) (layer "B.Cu") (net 2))
 (segment (start 128.667985 31.2645) (end 120.667985 31.2645) (width 0.25) (layer "B.Cu") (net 2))
 (segment (start 86.417985 67.7645) (end 95.917985 58.2645) (width 0.25) (layer "B.Cu") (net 2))
 (segment (start 128.917985 31.5145) (end 128.667985 31.2645) (width 0.25) (layer "B.Cu") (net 2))
 (segment (start 96.917985 57.2645) (end 92.667985 52.5145) (width 0.25) (layer "B.Cu") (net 2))
 (segment (start 127.417985 36.2645) (end 128.917985 34.7645) (width 0.25) (layer "B.Cu") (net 2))
 (segment (start 92.667985 52.5145) (end 91.917985 49.0145) (width 0.25) (layer "B.Cu") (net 2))
 (segment (start 128.917985 34.7645) (end 128.917985 31.5145) (width 0.25) (layer "B.Cu") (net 2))
 (segment (start 97.417985 45.7645) (end 127.417985 36.2645) (width 0.25) (layer "B.Cu") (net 2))
 (segment (start 111.417985 74.0145) (end 110.917985 73.0145) (width 0.25) (layer "B.Cu") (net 2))
 (segment (start 133.167985 67.7645) (end 133.167985 73.0145) (width 0.25) (layer "B.Cu") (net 2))
 (segment (start 104.167985 73.0145) (end 98.417985 70.5145) (width 0.25) (layer "B.Cu") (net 2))
 (segment (start 119.667985 32.7645) (end 119.667985 33.0145) (width 0.25) (layer "B.Cu") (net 2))
 (segment (start 120.667985 31.2645) (end 119.667985 32.7645) (width 0.25) (layer "B.Cu") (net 2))
 (segment (start 87.667985 52.5145) (end 86.667985 49.0145) (width 0.25) (layer "B.Cu") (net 5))
 (segment (start 117.417985 70.5145) (end 87.667985 52.5145) (width 0.25) (layer "B.Cu") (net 5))
 (segment (start 85.417985 52.7645) (end 85.167985 52.5145) (width 0.25) (layer "F.Cu") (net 4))
 (segment (start 85.167985 52.5145) (end 84.167985 49.0145) (width 0.25) (layer "F.Cu") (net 4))
 (segment (start 139.417985 70.5145) (end 85.417985 52.7645) (width 0.25) (layer "F.Cu") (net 4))
 (segment (start 82.417985 52.5145) (end 81.667985 49.0145) (width 0.25) (layer "F.Cu") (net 3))
 (segment (start 117.417985 93.0145) (end 100.417985 68.7645) (width 0.25) (layer "F.Cu") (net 3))
 (segment (start 100.417985 68.7645) (end 82.417985 52.5145) (width 0.25) (layer "F.Cu") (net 3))
 (segment (start 95.917985 35.5145) (end 85.417985 35.5145) (width 0.25) (layer "B.Cu") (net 11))
 (segment (start 126.167985 35.0145) (end 95.917985 35.5145) (width 0.25) (layer "B.Cu") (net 11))
 (segment (start 127.167985 33.0145) (end 126.417985 34.7645) (width 0.25) (layer "B.Cu") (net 11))
 (segment (start 85.417985 35.5145) (end 84.167985 33.7645) (width 0.25) (layer "B.Cu") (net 11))
 (segment (start 126.417985 34.7645) (end 126.167985 35.0145) (width 0.25) (layer "B.Cu") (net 11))
 (segment (start 123.917985 34.7645) (end 123.667985 35.0145) (width 0.25) (layer "F.Cu") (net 10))
 (segment (start 82.667985 35.5145) (end 81.667985 34.0145) (width 0.25) (layer "F.Cu") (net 10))
 (segment (start 81.667985 34.0145) (end 81.667985 33.7645) (width 0.25) (layer "F.Cu") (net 10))
 (segment (start 123.667985 35.0145) (end 95.917985 35.5145) (width 0.25) (layer "F.Cu") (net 10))
 (segment (start 95.917985 35.5145) (end 82.667985 35.5145) (width 0.25) (layer "F.Cu") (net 10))
 (segment (start 124.667985 33.0145) (end 123.917985 34.7645) (width 0.25) (layer "F.Cu") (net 10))
 (segment (start 128.917985 34.7645) (end 128.667985 35.0145) (width 0.25) (layer "F.Cu") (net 9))
 (segment (start 90.417985 47.2645) (end 89.417985 49.0145) (width 0.25) (layer "F.Cu") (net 9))
 (segment (start 128.917985 31.5145) (end 128.917985 34.7645) (width 0.25) (layer "F.Cu") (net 9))
 (segment (start 128.667985 35.0145) (end 90.417985 47.2645) (width 0.25) (layer "F.Cu") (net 9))
 (segment (start 128.667985 31.2645) (end 128.917985 31.5145) (width 0.25) (layer "F.Cu") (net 9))
 (segment (start 122.167985 33.0145) (end 122.167985 32.2645) (width 0.25) (layer "F.Cu") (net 9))
 (segment (start 122.167985 32.2645) (end 123.167985 31.2645) (width 0.25) (layer "F.Cu") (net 9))
 (segment (start 123.167985 31.2645) (end 128.667985 31.2645) (width 0.25) (layer "F.Cu") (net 9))
 (segment (start 77.667985 30.0145) (end 88.167985 30.0145) (width 0.25) (layer "F.Cu") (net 6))
 (segment (start 88.417985 30.2645) (end 89.417985 33.7645) (width 0.25) (layer "F.Cu") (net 6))
 (segment (start 77.417985 30.2645) (end 77.667985 30.0145) (width 0.25) (layer "F.Cu") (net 6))
 (segment (start 77.167985 36.2645) (end 77.417985 30.2645) (width 0.25) (layer "F.Cu") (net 6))
 (segment (start 88.167985 30.0145) (end 88.417985 30.2645) (width 0.25) (layer "F.Cu") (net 6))
 (via (at 77.167985 36.2645) (size 0.6) (drill 0.3) (layers "F.Cu" "B.Cu") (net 6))
 (segment (start 83.917985 70.5145) (end 77.417985 52.5145) (width 0.25) (layer "B.Cu") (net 6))
 (segment (start 77.417985 52.5145) (end 77.167985 36.2645) (width 0.25) (layer "B.Cu") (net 6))
 (segment (start 83.917985 75.5145) (end 82.167985 74.5145) (width 0.25) (layer "F.Cu") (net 7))
 (segment (start 77.667985 37.0145) (end 79.167985 33.7645) (width 0.25) (layer "F.Cu") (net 7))
 (segment (start 82.167985 74.5145) (end 77.417985 52.5145) (width 0.25) (layer "F.Cu") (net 7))
 (segment (start 77.417985 52.5145) (end 77.667985 37.0145) (width 0.25) (layer "F.Cu") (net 7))
 (segment (start 98.417985 75.5145) (end 94.167985 68.0145) (width 0.25) (layer "F.Cu") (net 8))
 (segment (start 79.917985 52.5145) (end 79.167985 49.0145) (width 0.25) (layer "F.Cu") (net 8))
 (segment (start 94.167985 68.0145) (end 94.167985 66.0145) (width 0.25) (layer "F.Cu") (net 8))
 (segment (start 94.167985 66.0145) (end 79.917985 52.5145) (width 0.25) (layer "F.Cu") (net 8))
 (segment (start 79.167985 37.0145) (end 77.417985 35.2645) (width 0.25) (layer "B.Cu") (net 1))
 (segment (start 119.417985 68.7645) (end 87.667985 37.0145) (width 0.25) (layer "B.Cu") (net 1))
 (segment (start 77.417985 35.2645) (end 77.417985 30.2645) (width 0.25) (layer "B.Cu") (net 1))
 (segment (start 77.667985 30.0145) (end 85.667985 30.0145) (width 0.25) (layer "B.Cu") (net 1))
 (segment (start 77.417985 30.2645) (end 77.667985 30.0145) (width 0.25) (layer "B.Cu") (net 1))
 (segment (start 87.667985 37.0145) (end 79.167985 37.0145) (width 0.25) (layer "B.Cu") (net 1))
 (segment (start 85.917985 30.2645) (end 86.667985 33.7645) (width 0.25) (layer "B.Cu") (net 1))
 (segment (start 85.667985 30.0145) (end 85.917985 30.2645) (width 0.25) (layer "B.Cu") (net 1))
 (segment (start 139.417985 93.0145) (end 119.417985 68.7645) (width 0.25) (layer "B.Cu") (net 1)))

